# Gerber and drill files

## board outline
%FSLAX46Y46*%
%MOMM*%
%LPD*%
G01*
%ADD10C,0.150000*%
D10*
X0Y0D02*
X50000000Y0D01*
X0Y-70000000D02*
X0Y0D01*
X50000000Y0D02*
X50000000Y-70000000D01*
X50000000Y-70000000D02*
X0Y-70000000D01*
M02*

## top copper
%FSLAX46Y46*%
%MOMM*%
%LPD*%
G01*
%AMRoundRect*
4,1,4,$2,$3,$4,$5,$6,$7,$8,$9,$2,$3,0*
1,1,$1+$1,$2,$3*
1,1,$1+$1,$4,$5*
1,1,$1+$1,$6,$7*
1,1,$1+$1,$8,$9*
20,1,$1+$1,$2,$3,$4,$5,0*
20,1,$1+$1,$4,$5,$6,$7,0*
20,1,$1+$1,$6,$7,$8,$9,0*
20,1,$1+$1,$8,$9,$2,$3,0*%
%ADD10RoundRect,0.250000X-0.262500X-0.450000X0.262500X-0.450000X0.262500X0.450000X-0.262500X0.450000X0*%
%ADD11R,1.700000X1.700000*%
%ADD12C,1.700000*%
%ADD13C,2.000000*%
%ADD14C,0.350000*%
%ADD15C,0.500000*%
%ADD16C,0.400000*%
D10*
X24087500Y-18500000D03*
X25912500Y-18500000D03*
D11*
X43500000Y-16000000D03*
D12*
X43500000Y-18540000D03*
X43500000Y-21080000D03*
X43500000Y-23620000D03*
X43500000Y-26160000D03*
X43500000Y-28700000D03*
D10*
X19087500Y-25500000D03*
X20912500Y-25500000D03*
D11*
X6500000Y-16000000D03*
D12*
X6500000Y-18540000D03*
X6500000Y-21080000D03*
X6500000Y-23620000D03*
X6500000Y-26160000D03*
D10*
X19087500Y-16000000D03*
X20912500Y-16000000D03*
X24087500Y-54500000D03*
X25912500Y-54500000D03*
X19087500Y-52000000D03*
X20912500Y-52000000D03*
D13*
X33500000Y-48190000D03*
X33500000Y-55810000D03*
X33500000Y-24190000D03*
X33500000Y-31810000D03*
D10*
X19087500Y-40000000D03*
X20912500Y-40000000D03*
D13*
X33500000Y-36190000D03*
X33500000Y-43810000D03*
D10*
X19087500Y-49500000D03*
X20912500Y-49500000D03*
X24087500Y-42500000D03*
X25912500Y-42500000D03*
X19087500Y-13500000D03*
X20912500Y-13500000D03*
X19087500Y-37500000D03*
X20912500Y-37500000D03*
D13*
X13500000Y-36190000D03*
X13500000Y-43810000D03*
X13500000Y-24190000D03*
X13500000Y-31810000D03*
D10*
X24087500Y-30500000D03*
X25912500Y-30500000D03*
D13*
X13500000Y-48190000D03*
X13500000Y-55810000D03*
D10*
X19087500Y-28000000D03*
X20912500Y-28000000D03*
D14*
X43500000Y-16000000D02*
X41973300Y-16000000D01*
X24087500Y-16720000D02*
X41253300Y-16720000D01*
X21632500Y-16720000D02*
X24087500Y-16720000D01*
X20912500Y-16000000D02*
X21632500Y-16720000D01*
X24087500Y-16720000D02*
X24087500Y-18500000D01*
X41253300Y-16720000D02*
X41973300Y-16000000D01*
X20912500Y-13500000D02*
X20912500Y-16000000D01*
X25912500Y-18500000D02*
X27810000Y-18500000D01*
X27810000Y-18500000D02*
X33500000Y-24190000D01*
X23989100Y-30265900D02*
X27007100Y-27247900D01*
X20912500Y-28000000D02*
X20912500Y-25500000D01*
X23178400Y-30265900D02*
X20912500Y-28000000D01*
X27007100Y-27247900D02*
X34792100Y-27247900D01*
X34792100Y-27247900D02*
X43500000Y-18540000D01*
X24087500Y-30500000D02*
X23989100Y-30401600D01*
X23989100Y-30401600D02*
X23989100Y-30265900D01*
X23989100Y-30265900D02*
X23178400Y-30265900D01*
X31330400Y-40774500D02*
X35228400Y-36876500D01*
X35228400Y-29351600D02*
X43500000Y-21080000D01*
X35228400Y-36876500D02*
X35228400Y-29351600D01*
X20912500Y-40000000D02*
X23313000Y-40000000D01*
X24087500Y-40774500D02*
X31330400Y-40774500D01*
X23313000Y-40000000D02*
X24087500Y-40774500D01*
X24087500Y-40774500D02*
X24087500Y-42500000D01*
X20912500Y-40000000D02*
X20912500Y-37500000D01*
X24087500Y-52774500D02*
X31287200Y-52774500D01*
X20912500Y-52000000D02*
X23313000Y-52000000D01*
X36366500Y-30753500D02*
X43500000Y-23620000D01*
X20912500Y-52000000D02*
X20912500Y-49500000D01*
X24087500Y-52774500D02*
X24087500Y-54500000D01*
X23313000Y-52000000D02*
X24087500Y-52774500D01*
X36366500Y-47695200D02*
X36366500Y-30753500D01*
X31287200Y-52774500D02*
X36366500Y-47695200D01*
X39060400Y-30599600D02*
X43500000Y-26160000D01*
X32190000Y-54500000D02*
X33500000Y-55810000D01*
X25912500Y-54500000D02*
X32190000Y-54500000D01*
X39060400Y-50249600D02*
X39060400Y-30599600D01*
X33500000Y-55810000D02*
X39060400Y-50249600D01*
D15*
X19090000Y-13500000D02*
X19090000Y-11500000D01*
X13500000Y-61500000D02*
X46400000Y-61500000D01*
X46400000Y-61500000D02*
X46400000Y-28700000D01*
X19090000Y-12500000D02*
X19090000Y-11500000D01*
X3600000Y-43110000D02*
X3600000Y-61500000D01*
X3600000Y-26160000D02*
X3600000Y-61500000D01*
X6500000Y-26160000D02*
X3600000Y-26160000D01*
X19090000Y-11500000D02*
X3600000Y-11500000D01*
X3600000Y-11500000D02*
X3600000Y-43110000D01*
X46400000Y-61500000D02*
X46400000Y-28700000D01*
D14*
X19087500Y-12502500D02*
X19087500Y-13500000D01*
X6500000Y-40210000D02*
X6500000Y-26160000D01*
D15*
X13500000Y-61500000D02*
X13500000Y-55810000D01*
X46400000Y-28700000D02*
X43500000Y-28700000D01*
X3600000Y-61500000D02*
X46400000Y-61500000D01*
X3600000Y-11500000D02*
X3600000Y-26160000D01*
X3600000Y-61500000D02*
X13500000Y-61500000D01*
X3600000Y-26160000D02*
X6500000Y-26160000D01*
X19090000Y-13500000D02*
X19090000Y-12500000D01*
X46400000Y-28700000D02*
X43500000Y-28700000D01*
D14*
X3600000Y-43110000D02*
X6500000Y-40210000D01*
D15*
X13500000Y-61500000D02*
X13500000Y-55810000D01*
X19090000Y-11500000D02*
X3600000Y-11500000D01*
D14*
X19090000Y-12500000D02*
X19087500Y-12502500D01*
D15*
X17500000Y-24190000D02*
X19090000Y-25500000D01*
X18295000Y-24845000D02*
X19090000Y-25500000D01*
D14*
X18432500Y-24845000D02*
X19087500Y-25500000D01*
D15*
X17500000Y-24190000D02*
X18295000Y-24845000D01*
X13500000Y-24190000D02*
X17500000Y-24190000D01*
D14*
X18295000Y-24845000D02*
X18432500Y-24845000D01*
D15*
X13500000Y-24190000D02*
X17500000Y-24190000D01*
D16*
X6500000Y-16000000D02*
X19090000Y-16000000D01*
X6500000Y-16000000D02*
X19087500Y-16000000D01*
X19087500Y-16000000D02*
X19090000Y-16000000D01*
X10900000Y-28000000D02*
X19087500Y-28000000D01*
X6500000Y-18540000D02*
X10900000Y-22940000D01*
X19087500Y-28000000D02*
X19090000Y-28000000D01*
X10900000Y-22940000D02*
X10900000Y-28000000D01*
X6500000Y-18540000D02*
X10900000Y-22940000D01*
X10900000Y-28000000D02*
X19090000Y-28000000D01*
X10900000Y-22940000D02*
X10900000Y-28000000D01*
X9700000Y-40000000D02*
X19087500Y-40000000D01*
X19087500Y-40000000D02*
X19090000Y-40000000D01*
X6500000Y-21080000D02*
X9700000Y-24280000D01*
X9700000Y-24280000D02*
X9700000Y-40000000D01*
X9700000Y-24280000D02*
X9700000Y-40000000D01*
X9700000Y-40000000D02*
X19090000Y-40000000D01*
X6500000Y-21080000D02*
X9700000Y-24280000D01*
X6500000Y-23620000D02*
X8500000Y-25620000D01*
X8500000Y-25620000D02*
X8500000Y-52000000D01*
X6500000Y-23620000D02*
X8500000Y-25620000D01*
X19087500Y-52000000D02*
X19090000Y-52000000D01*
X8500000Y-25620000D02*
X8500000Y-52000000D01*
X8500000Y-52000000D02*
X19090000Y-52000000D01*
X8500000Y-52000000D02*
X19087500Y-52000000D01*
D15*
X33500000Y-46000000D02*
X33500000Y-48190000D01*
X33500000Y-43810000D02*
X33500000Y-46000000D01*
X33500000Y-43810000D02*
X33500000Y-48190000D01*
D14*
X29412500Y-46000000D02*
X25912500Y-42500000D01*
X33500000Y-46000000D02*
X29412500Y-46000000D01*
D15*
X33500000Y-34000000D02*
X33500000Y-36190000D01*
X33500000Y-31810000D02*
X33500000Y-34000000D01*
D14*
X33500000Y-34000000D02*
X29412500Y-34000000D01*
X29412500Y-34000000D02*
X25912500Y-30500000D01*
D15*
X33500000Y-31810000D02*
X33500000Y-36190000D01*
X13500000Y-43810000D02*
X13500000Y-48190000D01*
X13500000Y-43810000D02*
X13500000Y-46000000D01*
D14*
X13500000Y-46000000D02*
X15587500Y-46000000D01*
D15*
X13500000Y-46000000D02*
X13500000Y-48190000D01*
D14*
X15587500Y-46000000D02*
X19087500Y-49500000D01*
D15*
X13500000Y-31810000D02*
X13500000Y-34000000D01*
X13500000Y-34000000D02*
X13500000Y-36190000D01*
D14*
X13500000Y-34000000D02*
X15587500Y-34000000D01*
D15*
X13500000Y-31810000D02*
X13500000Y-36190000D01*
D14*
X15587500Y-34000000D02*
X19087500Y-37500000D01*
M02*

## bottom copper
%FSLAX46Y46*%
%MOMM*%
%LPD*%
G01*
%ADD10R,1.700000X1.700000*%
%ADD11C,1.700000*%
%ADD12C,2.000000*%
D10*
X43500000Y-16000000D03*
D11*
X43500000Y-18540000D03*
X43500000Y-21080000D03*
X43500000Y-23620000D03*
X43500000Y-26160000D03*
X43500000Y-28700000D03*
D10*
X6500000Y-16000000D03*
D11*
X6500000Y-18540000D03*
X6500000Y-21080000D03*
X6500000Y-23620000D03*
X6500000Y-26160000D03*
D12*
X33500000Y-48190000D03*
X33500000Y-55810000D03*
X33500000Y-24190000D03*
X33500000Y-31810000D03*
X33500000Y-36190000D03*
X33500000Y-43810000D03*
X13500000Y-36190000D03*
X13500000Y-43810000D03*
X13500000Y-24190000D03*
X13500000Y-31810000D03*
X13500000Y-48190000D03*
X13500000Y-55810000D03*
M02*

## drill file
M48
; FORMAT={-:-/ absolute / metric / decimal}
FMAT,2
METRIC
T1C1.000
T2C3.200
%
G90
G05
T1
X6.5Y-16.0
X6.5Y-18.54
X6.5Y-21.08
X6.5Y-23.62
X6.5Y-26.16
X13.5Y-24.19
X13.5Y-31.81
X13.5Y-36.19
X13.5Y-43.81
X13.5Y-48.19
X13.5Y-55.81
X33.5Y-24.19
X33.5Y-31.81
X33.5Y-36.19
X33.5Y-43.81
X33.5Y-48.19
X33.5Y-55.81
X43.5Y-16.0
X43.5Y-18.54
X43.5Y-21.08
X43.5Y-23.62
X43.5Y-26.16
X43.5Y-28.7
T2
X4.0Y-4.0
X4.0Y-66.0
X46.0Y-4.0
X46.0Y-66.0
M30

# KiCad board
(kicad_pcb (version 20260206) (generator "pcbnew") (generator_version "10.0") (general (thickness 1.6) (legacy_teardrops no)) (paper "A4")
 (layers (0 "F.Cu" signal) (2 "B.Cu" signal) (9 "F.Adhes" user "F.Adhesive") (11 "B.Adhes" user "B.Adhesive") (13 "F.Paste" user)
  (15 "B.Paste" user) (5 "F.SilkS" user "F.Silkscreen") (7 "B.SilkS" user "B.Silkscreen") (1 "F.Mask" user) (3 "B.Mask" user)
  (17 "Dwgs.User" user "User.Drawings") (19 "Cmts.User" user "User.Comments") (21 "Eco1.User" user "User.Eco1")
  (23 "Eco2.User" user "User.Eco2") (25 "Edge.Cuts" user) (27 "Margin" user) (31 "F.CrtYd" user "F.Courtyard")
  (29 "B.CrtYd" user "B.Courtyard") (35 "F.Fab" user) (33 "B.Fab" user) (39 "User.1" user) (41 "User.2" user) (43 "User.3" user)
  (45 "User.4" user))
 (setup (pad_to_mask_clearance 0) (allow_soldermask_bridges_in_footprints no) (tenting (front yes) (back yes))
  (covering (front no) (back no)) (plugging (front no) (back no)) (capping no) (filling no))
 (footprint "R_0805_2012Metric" (layer "F.Cu") (at 25 18.5)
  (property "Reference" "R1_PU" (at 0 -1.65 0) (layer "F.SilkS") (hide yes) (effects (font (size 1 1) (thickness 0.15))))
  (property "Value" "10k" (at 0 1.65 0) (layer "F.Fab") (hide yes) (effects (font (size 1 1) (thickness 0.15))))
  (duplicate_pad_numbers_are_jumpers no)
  (pad "1" smd roundrect (at -0.9125 0) (size 1.025 1.4) (layers "F.Cu" "F.Mask" "F.Paste") (roundrect_rratio 0.243902) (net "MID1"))
  (pad "2" smd roundrect (at 0.9125 0) (size 1.025 1.4) (layers "F.Cu" "F.Mask" "F.Paste") (roundrect_rratio 0.243902) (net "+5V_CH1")))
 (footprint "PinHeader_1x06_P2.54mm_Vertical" (layer "F.Cu") (at 43.5 16)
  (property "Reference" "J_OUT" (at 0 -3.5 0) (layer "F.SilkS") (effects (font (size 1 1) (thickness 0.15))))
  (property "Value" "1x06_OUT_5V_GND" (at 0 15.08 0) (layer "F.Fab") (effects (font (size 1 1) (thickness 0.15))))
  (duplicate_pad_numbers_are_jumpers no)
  (pad "1" thru_hole rect (at 0 0) (size 1.7 1.7) (drill 1) (layers "*.Cu" "F.Mask") (remove_unused_layers no) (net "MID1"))
  (pad "2" thru_hole circle (at 0 2.54) (size 1.7 1.7) (drill 1) (layers "*.Cu" "F.Mask") (remove_unused_layers no) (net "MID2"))
  (pad "3" thru_hole circle (at 0 5.08) (size 1.7 1.7) (drill 1) (layers "*.Cu" "F.Mask") (remove_unused_layers no) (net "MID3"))
  (pad "4" thru_hole circle (at 0 7.62) (size 1.7 1.7) (drill 1) (layers "*.Cu" "F.Mask") (remove_unused_layers no) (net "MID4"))
  (pad "5" thru_hole circle (at 0 10.16) (size 1.7 1.7) (drill 1) (layers "*.Cu" "F.Mask") (remove_unused_layers no) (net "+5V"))
  (pad "6" thru_hole circle (at 0 12.7) (size 1.7 1.7) (drill 1) (layers "*.Cu" "F.Mask") (remove_unused_layers no) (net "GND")))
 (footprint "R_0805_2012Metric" (layer "F.Cu") (at 20 25.5)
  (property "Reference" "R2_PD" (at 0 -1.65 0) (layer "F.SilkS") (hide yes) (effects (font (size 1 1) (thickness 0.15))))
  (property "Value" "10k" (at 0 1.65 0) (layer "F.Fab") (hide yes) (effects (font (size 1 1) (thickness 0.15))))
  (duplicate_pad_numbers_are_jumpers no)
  (pad "1" smd roundrect (at -0.9125 0) (size 1.025 1.4) (layers "F.Cu" "F.Mask" "F.Paste") (roundrect_rratio 0.243902) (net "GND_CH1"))
  (pad "2" smd roundrect (at 0.9125 0) (size 1.025 1.4) (layers "F.Cu" "F.Mask" "F.Paste") (roundrect_rratio 0.243902) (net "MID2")))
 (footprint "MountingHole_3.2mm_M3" (layer "F.Cu") (at 46 4)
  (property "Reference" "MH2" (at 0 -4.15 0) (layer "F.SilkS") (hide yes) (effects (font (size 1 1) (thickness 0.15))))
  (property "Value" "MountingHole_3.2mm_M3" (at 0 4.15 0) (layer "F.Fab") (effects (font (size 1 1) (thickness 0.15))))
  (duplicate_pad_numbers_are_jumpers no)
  (pad "" np_thru_hole circle (at 0 0) (size 3.2 3.2) (drill 3.2) (layers "*.Cu")))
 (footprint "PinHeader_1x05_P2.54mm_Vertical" (layer "F.Cu") (at 6.5 16)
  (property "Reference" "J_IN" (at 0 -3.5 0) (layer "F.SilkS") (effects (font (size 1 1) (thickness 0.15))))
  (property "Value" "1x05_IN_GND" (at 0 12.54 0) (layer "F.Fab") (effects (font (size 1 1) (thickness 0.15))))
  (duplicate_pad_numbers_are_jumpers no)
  (pad "1" thru_hole rect (at 0 0) (size 1.7 1.7) (drill 1) (layers "*.Cu" "F.Mask") (remove_unused_layers no) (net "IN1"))
  (pad "2" thru_hole circle (at 0 2.54) (size 1.7 1.7) (drill 1) (layers "*.Cu" "F.Mask") (remove_unused_layers no) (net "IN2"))
  (pad "3" thru_hole circle (at 0 5.08) (size 1.7 1.7) (drill 1) (layers "*.Cu" "F.Mask") (remove_unused_layers no) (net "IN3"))
  (pad "4" thru_hole circle (at 0 7.62) (size 1.7 1.7) (drill 1) (layers "*.Cu" "F.Mask") (remove_unused_layers no) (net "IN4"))
  (pad "5" thru_hole circle (at 0 10.16) (size 1.7 1.7) (drill 1) (layers "*.Cu" "F.Mask") (remove_unused_layers no) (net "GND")))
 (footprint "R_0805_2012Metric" (layer "F.Cu") (at 20 16)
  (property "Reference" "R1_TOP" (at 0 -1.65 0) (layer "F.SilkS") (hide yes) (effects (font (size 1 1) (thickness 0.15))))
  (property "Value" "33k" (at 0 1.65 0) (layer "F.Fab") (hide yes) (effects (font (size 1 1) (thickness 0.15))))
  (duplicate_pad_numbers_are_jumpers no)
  (pad "1" smd roundrect (at -0.9125 0) (size 1.025 1.4) (layers "F.Cu" "F.Mask" "F.Paste") (roundrect_rratio 0.243902) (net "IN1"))
  (pad "2" smd roundrect (at 0.9125 0) (size 1.025 1.4) (layers "F.Cu" "F.Mask" "F.Paste") (roundrect_rratio 0.243902) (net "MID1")))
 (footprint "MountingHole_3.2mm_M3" (layer "F.Cu") (at 4 4)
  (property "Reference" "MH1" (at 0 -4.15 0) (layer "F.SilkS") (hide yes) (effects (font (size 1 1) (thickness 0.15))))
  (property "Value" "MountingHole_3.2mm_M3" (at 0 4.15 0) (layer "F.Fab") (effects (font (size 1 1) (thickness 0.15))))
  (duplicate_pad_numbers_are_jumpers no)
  (pad "" np_thru_hole circle (at 0 0) (size 3.2 3.2) (drill 3.2) (layers "*.Cu")))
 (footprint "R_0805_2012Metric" (layer "F.Cu") (at 25 54.5)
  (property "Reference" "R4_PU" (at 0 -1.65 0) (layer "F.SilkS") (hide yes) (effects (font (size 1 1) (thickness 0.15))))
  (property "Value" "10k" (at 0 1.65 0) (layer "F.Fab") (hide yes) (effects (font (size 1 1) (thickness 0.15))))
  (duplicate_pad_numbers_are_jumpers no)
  (pad "1" smd roundrect (at -0.9125 0) (size 1.025 1.4) (layers "F.Cu" "F.Mask" "F.Paste") (roundrect_rratio 0.243902) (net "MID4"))
  (pad "2" smd roundrect (at 0.9125 0) (size 1.025 1.4) (layers "F.Cu" "F.Mask" "F.Paste") (roundrect_rratio 0.243902) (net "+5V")))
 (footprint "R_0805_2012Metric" (layer "F.Cu") (at 20 52)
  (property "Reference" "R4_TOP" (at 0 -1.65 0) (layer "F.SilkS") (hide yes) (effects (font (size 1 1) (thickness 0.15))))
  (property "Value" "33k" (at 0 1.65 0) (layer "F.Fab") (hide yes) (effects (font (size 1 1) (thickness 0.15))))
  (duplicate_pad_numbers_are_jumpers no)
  (pad "1" smd roundrect (at -0.9125 0) (size 1.025 1.4) (layers "F.Cu" "F.Mask" "F.Paste") (roundrect_rratio 0.243902) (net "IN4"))
  (pad "2" smd roundrect (at 0.9125 0) (size 1.025 1.4) (layers "F.Cu" "F.Mask" "F.Paste") (roundrect_rratio 0.243902) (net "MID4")))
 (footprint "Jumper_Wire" (layer "F.Cu") (at 33.5 52 90)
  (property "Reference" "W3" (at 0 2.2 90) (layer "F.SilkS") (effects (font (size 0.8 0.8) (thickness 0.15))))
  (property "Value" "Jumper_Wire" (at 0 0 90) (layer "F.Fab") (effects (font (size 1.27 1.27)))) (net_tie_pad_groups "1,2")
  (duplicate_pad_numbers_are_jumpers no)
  (pad "1" thru_hole circle (at 3.81 0) (size 2 2) (drill 1) (layers "*.Cu" "F.Mask") (remove_unused_layers no) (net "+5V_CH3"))
  (pad "2" thru_hole circle (at -3.81 0) (size 2 2) (drill 1) (layers "*.Cu" "F.Mask") (remove_unused_layers no) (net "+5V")))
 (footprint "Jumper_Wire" (layer "F.Cu") (at 33.5 28 90)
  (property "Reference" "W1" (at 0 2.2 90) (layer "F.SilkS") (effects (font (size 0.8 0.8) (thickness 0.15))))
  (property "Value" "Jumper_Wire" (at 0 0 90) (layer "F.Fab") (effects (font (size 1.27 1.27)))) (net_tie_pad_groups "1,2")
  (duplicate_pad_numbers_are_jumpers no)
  (pad "1" thru_hole circle (at 3.81 0) (size 2 2) (drill 1) (layers "*.Cu" "F.Mask") (remove_unused_layers no) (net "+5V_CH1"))
  (pad "2" thru_hole circle (at -3.81 0) (size 2 2) (drill 1) (layers "*.Cu" "F.Mask") (remove_unused_layers no) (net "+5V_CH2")))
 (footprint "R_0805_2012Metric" (layer "F.Cu") (at 20 40)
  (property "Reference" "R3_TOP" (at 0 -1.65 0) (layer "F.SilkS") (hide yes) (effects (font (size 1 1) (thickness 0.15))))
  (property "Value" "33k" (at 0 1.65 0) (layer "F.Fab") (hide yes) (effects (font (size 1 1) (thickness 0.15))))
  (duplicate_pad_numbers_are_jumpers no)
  (pad "1" smd roundrect (at -0.9125 0) (size 1.025 1.4) (layers "F.Cu" "F.Mask" "F.Paste") (roundrect_rratio 0.243902) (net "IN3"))
  (pad "2" smd roundrect (at 0.9125 0) (size 1.025 1.4) (layers "F.Cu" "F.Mask" "F.Paste") (roundrect_rratio 0.243902) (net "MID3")))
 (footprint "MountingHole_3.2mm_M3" (layer "F.Cu") (at 46 66)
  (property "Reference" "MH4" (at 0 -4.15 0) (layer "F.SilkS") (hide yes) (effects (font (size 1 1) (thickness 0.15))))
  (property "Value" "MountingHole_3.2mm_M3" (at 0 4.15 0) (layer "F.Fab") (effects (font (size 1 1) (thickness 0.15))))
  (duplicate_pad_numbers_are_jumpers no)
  (pad "" np_thru_hole circle (at 0 0) (size 3.2 3.2) (drill 3.2) (layers "*.Cu")))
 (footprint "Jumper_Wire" (layer "F.Cu") (at 33.5 40 90)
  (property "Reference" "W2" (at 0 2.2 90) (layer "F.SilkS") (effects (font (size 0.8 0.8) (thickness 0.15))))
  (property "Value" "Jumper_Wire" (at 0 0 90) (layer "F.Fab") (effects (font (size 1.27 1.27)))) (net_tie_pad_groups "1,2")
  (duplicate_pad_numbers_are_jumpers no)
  (pad "1" thru_hole circle (at 3.81 0) (size 2 2) (drill 1) (layers "*.Cu" "F.Mask") (remove_unused_layers no) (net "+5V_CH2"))
  (pad "2" thru_hole circle (at -3.81 0) (size 2 2) (drill 1) (layers "*.Cu" "F.Mask") (remove_unused_layers no) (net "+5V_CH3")))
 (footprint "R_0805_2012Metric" (layer "F.Cu") (at 20 49.5)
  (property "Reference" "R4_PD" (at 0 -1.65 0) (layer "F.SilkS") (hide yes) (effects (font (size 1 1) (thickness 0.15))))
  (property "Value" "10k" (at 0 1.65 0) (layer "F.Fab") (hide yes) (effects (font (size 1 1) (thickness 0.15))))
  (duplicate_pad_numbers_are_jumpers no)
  (pad "1" smd roundrect (at -0.9125 0) (size 1.025 1.4) (layers "F.Cu" "F.Mask" "F.Paste") (roundrect_rratio 0.243902) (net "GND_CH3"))
  (pad "2" smd roundrect (at 0.9125 0) (size 1.025 1.4) (layers "F.Cu" "F.Mask" "F.Paste") (roundrect_rratio 0.243902) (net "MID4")))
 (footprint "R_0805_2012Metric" (layer "F.Cu") (at 25 42.5)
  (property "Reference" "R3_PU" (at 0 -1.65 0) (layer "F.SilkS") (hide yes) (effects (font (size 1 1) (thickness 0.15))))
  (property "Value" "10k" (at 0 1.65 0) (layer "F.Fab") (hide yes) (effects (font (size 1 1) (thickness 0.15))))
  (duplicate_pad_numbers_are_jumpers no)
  (pad "1" smd roundrect (at -0.9125 0) (size 1.025 1.4) (layers "F.Cu" "F.Mask" "F.Paste") (roundrect_rratio 0.243902) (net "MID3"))
  (pad "2" smd roundrect (at 0.9125 0) (size 1.025 1.4) (layers "F.Cu" "F.Mask" "F.Paste") (roundrect_rratio 0.243902) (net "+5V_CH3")))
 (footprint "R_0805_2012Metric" (layer "F.Cu") (at 20 13.5)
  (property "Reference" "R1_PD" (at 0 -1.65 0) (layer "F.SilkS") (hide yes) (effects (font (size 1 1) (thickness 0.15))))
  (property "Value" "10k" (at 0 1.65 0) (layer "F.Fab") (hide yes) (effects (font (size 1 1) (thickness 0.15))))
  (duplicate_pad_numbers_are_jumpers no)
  (pad "1" smd roundrect (at -0.9125 0) (size 1.025 1.4) (layers "F.Cu" "F.Mask" "F.Paste") (roundrect_rratio 0.243902) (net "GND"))
  (pad "2" smd roundrect (at 0.9125 0) (size 1.025 1.4) (layers "F.Cu" "F.Mask" "F.Paste") (roundrect_rratio 0.243902) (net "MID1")))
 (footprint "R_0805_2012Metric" (layer "F.Cu") (at 20 37.5)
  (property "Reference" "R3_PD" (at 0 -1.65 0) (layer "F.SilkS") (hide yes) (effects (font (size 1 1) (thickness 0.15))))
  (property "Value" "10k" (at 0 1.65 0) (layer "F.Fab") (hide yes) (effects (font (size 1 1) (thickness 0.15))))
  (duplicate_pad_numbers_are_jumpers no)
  (pad "1" smd roundrect (at -0.9125 0) (size 1.025 1.4) (layers "F.Cu" "F.Mask" "F.Paste") (roundrect_rratio 0.243902) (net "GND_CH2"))
  (pad "2" smd roundrect (at 0.9125 0) (size 1.025 1.4) (layers "F.Cu" "F.Mask" "F.Paste") (roundrect_rratio 0.243902) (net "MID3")))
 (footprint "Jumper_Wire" (layer "F.Cu") (at 13.5 40 90)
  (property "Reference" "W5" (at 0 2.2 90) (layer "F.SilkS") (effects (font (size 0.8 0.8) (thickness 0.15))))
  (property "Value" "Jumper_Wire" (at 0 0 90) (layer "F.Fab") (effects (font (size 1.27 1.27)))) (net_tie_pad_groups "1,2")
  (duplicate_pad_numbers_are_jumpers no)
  (pad "1" thru_hole circle (at 3.81 0) (size 2 2) (drill 1) (layers "*.Cu" "F.Mask") (remove_unused_layers no) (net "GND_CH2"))
  (pad "2" thru_hole circle (at -3.81 0) (size 2 2) (drill 1) (layers "*.Cu" "F.Mask") (remove_unused_layers no) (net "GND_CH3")))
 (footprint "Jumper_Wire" (layer "F.Cu") (at 13.5 28 90)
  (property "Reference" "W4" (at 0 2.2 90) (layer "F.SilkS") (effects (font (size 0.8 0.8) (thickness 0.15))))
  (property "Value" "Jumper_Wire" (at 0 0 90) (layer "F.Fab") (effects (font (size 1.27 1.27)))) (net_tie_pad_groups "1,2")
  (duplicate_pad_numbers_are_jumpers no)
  (pad "1" thru_hole circle (at 3.81 0) (size 2 2) (drill 1) (layers "*.Cu" "F.Mask") (remove_unused_layers no) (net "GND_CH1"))
  (pad "2" thru_hole circle (at -3.81 0) (size 2 2) (drill 1) (layers "*.Cu" "F.Mask") (remove_unused_layers no) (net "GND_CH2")))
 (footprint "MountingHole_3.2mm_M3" (layer "F.Cu") (at 4 66)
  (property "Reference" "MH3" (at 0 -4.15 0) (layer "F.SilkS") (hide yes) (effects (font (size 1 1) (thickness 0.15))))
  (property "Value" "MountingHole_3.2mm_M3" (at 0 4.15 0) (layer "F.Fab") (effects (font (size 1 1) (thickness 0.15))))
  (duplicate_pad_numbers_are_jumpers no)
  (pad "" np_thru_hole circle (at 0 0) (size 3.2 3.2) (drill 3.2) (layers "*.Cu")))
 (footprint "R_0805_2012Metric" (layer "F.Cu") (at 25 30.5)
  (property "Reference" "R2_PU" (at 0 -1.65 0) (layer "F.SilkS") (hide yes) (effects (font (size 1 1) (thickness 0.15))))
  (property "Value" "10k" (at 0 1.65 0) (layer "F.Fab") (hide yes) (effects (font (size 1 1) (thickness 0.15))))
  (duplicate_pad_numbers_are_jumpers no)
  (pad "1" smd roundrect (at -0.9125 0) (size 1.025 1.4) (layers "F.Cu" "F.Mask" "F.Paste") (roundrect_rratio 0.243902) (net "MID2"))
  (pad "2" smd roundrect (at 0.9125 0) (size 1.025 1.4) (layers "F.Cu" "F.Mask" "F.Paste") (roundrect_rratio 0.243902) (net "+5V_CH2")))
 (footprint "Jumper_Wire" (layer "F.Cu") (at 13.5 52 90)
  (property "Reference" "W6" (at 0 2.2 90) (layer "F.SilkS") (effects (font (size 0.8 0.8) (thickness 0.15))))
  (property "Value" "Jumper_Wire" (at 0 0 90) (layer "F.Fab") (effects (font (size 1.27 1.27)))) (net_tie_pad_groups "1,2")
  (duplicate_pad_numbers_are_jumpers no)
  (pad "1" thru_hole circle (at 3.81 0) (size 2 2) (drill 1) (layers "*.Cu" "F.Mask") (remove_unused_layers no) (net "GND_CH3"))
  (pad "2" thru_hole circle (at -3.81 0) (size 2 2) (drill 1) (layers "*.Cu" "F.Mask") (remove_unused_layers no) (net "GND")))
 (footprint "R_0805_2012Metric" (layer "F.Cu") (at 20 28)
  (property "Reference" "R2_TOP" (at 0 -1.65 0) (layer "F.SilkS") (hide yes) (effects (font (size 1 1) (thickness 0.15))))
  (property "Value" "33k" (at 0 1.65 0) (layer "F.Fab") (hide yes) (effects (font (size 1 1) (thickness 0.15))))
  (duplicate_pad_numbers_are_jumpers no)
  (pad "1" smd roundrect (at -0.9125 0) (size 1.025 1.4) (layers "F.Cu" "F.Mask" "F.Paste") (roundrect_rratio 0.243902) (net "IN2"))
  (pad "2" smd roundrect (at 0.9125 0) (size 1.025 1.4) (layers "F.Cu" "F.Mask" "F.Paste") (roundrect_rratio 0.243902) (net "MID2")))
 (gr_line (start 0 0) (end 50 0) (stroke (width 0.15) (type default)) (layer "Edge.Cuts"))
 (gr_line (start 0 70) (end 0 0) (stroke (width 0.15) (type default)) (layer "Edge.Cuts"))
 (gr_line (start 50 0) (end 50 70) (stroke (width 0.15) (type default)) (layer "Edge.Cuts"))
 (gr_line (start 50 70) (end 0 70) (stroke (width 0.15) (type default)) (layer "Edge.Cuts"))
 (segment (start 43.5 16) (end 41.9733 16) (width 0.35) (layer "F.Cu") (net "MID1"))
 (segment (start 24.0875 16.72) (end 41.2533 16.72) (width 0.35) (layer "F.Cu") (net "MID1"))
 (segment (start 21.6325 16.72) (end 24.0875 16.72) (width 0.35) (layer "F.Cu") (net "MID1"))
 (segment (start 20.9125 16) (end 21.6325 16.72) (width 0.35) (layer "F.Cu") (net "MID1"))
 (segment (start 24.0875 16.72) (end 24.0875 18.5) (width 0.35) (layer "F.Cu") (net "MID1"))
 (segment (start 41.2533 16.72) (end 41.9733 16) (width 0.35) (layer "F.Cu") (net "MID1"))
 (segment (start 20.9125 13.5) (end 20.9125 16) (width 0.35) (layer "F.Cu") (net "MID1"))
 (segment (start 25.9125 18.5) (end 27.81 18.5) (width 0.35) (layer "F.Cu") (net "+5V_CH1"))
 (segment (start 27.81 18.5) (end 33.5 24.19) (width 0.35) (layer "F.Cu") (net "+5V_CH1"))
 (segment (start 23.9891 30.2659) (end 27.0071 27.2479) (width 0.35) (layer "F.Cu") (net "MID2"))
 (segment (start 20.9125 28) (end 20.9125 25.5) (width 0.35) (layer "F.Cu") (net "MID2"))
 (segment (start 23.1784 30.2659) (end 20.9125 28) (width 0.35) (layer "F.Cu") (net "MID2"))
 (segment (start 27.0071 27.2479) (end 34.7921 27.2479) (width 0.35) (layer "F.Cu") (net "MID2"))
 (segment (start 34.7921 27.2479) (end 43.5 18.54) (width 0.35) (layer "F.Cu") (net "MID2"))
 (segment (start 24.0875 30.5) (end 23.9891 30.4016) (width 0.35) (layer "F.Cu") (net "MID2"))
 (segment (start 23.9891 30.4016) (end 23.9891 30.2659) (width 0.35) (layer "F.Cu") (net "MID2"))
 (segment (start 23.9891 30.2659) (end 23.1784 30.2659) (width 0.35) (layer "F.Cu") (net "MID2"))
 (segment (start 31.3304 40.7745) (end 35.2284 36.8765) (width 0.35) (layer "F.Cu") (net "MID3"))
 (segment (start 35.2284 29.3516) (end 43.5 21.08) (width 0.35) (layer "F.Cu") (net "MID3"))
 (segment (start 35.2284 36.8765) (end 35.2284 29.3516) (width 0.35) (layer "F.Cu") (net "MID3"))
 (segment (start 20.9125 40) (end 23.313 40) (width 0.35) (layer "F.Cu") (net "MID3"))
 (segment (start 24.0875 40.7745) (end 31.3304 40.7745) (width 0.35) (layer "F.Cu") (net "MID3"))
 (segment (start 23.313 40) (end 24.0875 40.7745) (width 0.35) (layer "F.Cu") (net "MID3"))
 (segment (start 24.0875 40.7745) (end 24.0875 42.5) (width 0.35) (layer "F.Cu") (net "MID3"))
 (segment (start 20.9125 40) (end 20.9125 37.5) (width 0.35) (layer "F.Cu") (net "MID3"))
 (segment (start 24.0875 52.7745) (end 31.2872 52.7745) (width 0.35) (layer "F.Cu") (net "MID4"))
 (segment (start 20.9125 52) (end 23.313 52) (width 0.35) (layer "F.Cu") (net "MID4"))
 (segment (start 36.3665 30.7535) (end 43.5 23.62) (width 0.35) (layer "F.Cu") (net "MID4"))
 (segment (start 20.9125 52) (end 20.9125 49.5) (width 0.35) (layer "F.Cu") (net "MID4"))
 (segment (start 24.0875 52.7745) (end 24.0875 54.5) (width 0.35) (layer "F.Cu") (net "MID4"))
 (segment (start 23.313 52) (end 24.0875 52.7745) (width 0.35) (layer "F.Cu") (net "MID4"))
 (segment (start 36.3665 47.6952) (end 36.3665 30.7535) (width 0.35) (layer "F.Cu") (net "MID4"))
 (segment (start 31.2872 52.7745) (end 36.3665 47.6952) (width 0.35) (layer "F.Cu") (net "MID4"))
 (segment (start 39.0604 30.5996) (end 43.5 26.16) (width 0.35) (layer "F.Cu") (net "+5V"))
 (segment (start 32.19 54.5) (end 33.5 55.81) (width 0.35) (layer "F.Cu") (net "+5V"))
 (segment (start 25.9125 54.5) (end 32.19 54.5) (width 0.35) (layer "F.Cu") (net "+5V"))
 (segment (start 39.0604 50.2496) (end 39.0604 30.5996) (width 0.35) (layer "F.Cu") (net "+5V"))
 (segment (start 33.5 55.81) (end 39.0604 50.2496) (width 0.35) (layer "F.Cu") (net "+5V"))
 (segment (start 19.09 13.5) (end 19.09 11.5) (width 0.5) (layer "F.Cu") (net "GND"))
 (segment (start 13.5 61.5) (end 46.4 61.5) (width 0.5) (layer "F.Cu") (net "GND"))
 (segment (start 46.4 61.5) (end 46.4 28.7) (width 0.5) (layer "F.Cu") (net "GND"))
 (segment (start 19.09 12.5) (end 19.09 11.5) (width 0.5) (layer "F.Cu") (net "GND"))
 (segment (start 3.6 43.11) (end 3.6 61.5) (width 0.5) (layer "F.Cu") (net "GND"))
 (segment (start 3.6 26.16) (end 3.6 61.5) (width 0.5) (layer "F.Cu") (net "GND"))
 (segment (start 6.5 26.16) (end 3.6 26.16) (width 0.5) (layer "F.Cu") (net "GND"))
 (segment (start 19.09 11.5) (end 3.6 11.5) (width 0.5) (layer "F.Cu") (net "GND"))
 (segment (start 3.6 11.5) (end 3.6 43.11) (width 0.5) (layer "F.Cu") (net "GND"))
 (segment (start 46.4 61.5) (end 46.4 28.7) (width 0.5) (layer "F.Cu") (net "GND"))
 (segment (start 19.0875 12.5025) (end 19.0875 13.5) (width 0.35) (layer "F.Cu") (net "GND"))
 (segment (start 6.5 40.21) (end 6.5 26.16) (width 0.35) (layer "F.Cu") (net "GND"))
 (segment (start 13.5 61.5) (end 13.5 55.81) (width 0.5) (layer "F.Cu") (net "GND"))
 (segment (start 46.4 28.7) (end 43.5 28.7) (width 0.5) (layer "F.Cu") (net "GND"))
 (segment (start 3.6 61.5) (end 46.4 61.5) (width 0.5) (layer "F.Cu") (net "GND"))
 (segment (start 3.6 11.5) (end 3.6 26.16) (width 0.5) (layer "F.Cu") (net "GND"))
 (segment (start 3.6 61.5) (end 13.5 61.5) (width 0.5) (layer "F.Cu") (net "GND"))
 (segment (start 3.6 26.16) (end 6.5 26.16) (width 0.5) (layer "F.Cu") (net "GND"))
 (segment (start 19.09 13.5) (end 19.09 12.5) (width 0.5) (layer "F.Cu") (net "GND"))
 (segment (start 46.4 28.7) (end 43.5 28.7) (width 0.5) (layer "F.Cu") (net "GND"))
 (segment (start 3.6 43.11) (end 6.5 40.21) (width 0.35) (layer "F.Cu") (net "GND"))
 (segment (start 13.5 61.5) (end 13.5 55.81) (width 0.5) (layer "F.Cu") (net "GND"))
 (segment (start 19.09 11.5) (end 3.6 11.5) (width 0.5) (layer "F.Cu") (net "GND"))
 (segment (start 19.09 12.5) (end 19.0875 12.5025) (width 0.35) (layer "F.Cu") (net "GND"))
 (segment (start 17.5 24.19) (end 19.09 25.5) (width 0.5) (layer "F.Cu") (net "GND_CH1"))
 (segment (start 18.295 24.845) (end 19.09 25.5) (width 0.5) (layer "F.Cu") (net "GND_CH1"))
 (segment (start 18.4325 24.845) (end 19.0875 25.5) (width 0.35) (layer "F.Cu") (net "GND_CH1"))
 (segment (start 17.5 24.19) (end 18.295 24.845) (width 0.5) (layer "F.Cu") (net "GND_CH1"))
 (segment (start 13.5 24.19) (end 17.5 24.19) (width 0.5) (layer "F.Cu") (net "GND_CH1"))
 (segment (start 18.295 24.845) (end 18.4325 24.845) (width 0.35) (layer "F.Cu") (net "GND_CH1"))
 (segment (start 13.5 24.19) (end 17.5 24.19) (width 0.5) (layer "F.Cu") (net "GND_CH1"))
 (segment (start 6.5 16) (end 19.09 16) (width 0.4) (layer "F.Cu") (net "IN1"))
 (segment (start 6.5 16) (end 19.0875 16) (width 0.4) (layer "F.Cu") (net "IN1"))
 (segment (start 19.0875 16) (end 19.09 16) (width 0.4) (layer "F.Cu") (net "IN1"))
 (segment (start 10.9 28) (end 19.0875 28) (width 0.4) (layer "F.Cu") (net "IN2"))
 (segment (start 6.5 18.54) (end 10.9 22.94) (width 0.4) (layer "F.Cu") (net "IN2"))
 (segment (start 19.0875 28) (end 19.09 28) (width 0.4) (layer "F.Cu") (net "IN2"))
 (segment (start 10.9 22.94) (end 10.9 28) (width 0.4) (layer "F.Cu") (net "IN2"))
 (segment (start 6.5 18.54) (end 10.9 22.94) (width 0.4) (layer "F.Cu") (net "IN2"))
 (segment (start 10.9 28) (end 19.09 28) (width 0.4) (layer "F.Cu") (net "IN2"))
 (segment (start 10.9 22.94) (end 10.9 28) (width 0.4) (layer "F.Cu") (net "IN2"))
 (segment (start 9.7 40) (end 19.0875 40) (width 0.4) (layer "F.Cu") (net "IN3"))
 (segment (start 19.0875 40) (end 19.09 40) (width 0.4) (layer "F.Cu") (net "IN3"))
 (segment (start 6.5 21.08) (end 9.7 24.28) (width 0.4) (layer "F.Cu") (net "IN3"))
 (segment (start 9.7 24.28) (end 9.7 40) (width 0.4) (layer "F.Cu") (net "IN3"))
 (segment (start 9.7 24.28) (end 9.7 40) (width 0.4) (layer "F.Cu") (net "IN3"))
 (segment (start 9.7 40) (end 19.09 40) (width 0.4) (layer "F.Cu") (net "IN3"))
 (segment (start 6.5 21.08) (end 9.7 24.28) (width 0.4) (layer "F.Cu") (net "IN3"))
 (segment (start 6.5 23.62) (end 8.5 25.62) (width 0.4) (layer "F.Cu") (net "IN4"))
 (segment (start 8.5 25.62) (end 8.5 52) (width 0.4) (layer "F.Cu") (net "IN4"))
 (segment (start 6.5 23.62) (end 8.5 25.62) (width 0.4) (layer "F.Cu") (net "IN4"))
 (segment (start 19.0875 52) (end 19.09 52) (width 0.4) (layer "F.Cu") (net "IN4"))
 (segment (start 8.5 25.62) (end 8.5 52) (width 0.4) (layer "F.Cu") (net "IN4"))
 (segment (start 8.5 52) (end 19.09 52) (width 0.4) (layer "F.Cu") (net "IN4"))
 (segment (start 8.5 52) (end 19.0875 52) (width 0.4) (layer "F.Cu") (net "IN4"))
 (segment (start 33.5 46) (end 33.5 48.19) (width 0.5) (layer "F.Cu") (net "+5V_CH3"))
 (segment (start 33.5 43.81) (end 33.5 46) (width 0.5) (layer "F.Cu") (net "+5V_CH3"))
 (segment (start 33.5 43.81) (end 33.5 48.19) (width 0.5) (layer "F.Cu") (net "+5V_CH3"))
 (segment (start 29.4125 46) (end 25.9125 42.5) (width 0.35) (layer "F.Cu") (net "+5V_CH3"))
 (segment (start 33.5 46) (end 29.4125 46) (width 0.35) (layer "F.Cu") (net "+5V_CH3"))
 (segment (start 33.5 34) (end 33.5 36.19) (width 0.5) (layer "F.Cu") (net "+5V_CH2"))
 (segment (start 33.5 31.81) (end 33.5 34) (width 0.5) (layer "F.Cu") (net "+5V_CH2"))
 (segment (start 33.5 34) (end 29.4125 34) (width 0.35) (layer "F.Cu") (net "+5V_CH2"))
 (segment (start 29.4125 34) (end 25.9125 30.5) (width 0.35) (layer "F.Cu") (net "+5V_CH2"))
 (segment (start 33.5 31.81) (end 33.5 36.19) (width 0.5) (layer "F.Cu") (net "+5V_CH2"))
 (segment (start 13.5 43.81) (end 13.5 48.19) (width 0.5) (layer "F.Cu") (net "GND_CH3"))
 (segment (start 13.5 43.81) (end 13.5 46) (width 0.5) (layer "F.Cu") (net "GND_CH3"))
 (segment (start 13.5 46) (end 15.5875 46) (width 0.35) (layer "F.Cu") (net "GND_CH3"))
 (segment (start 13.5 46) (end 13.5 48.19) (width 0.5) (layer "F.Cu") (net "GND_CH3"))
 (segment (start 15.5875 46) (end 19.0875 49.5) (width 0.35) (layer "F.Cu") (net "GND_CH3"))
 (segment (start 13.5 31.81) (end 13.5 34) (width 0.5) (layer "F.Cu") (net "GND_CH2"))
 (segment (start 13.5 34) (end 13.5 36.19) (width 0.5) (layer "F.Cu") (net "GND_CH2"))
 (segment (start 13.5 34) (end 15.5875 34) (width 0.35) (layer "F.Cu") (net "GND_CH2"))
 (segment (start 13.5 31.81) (end 13.5 36.19) (width 0.5) (layer "F.Cu") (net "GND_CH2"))
 (segment (start 15.5875 34) (end 19.0875 37.5) (width 0.35) (layer "F.Cu") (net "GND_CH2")))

